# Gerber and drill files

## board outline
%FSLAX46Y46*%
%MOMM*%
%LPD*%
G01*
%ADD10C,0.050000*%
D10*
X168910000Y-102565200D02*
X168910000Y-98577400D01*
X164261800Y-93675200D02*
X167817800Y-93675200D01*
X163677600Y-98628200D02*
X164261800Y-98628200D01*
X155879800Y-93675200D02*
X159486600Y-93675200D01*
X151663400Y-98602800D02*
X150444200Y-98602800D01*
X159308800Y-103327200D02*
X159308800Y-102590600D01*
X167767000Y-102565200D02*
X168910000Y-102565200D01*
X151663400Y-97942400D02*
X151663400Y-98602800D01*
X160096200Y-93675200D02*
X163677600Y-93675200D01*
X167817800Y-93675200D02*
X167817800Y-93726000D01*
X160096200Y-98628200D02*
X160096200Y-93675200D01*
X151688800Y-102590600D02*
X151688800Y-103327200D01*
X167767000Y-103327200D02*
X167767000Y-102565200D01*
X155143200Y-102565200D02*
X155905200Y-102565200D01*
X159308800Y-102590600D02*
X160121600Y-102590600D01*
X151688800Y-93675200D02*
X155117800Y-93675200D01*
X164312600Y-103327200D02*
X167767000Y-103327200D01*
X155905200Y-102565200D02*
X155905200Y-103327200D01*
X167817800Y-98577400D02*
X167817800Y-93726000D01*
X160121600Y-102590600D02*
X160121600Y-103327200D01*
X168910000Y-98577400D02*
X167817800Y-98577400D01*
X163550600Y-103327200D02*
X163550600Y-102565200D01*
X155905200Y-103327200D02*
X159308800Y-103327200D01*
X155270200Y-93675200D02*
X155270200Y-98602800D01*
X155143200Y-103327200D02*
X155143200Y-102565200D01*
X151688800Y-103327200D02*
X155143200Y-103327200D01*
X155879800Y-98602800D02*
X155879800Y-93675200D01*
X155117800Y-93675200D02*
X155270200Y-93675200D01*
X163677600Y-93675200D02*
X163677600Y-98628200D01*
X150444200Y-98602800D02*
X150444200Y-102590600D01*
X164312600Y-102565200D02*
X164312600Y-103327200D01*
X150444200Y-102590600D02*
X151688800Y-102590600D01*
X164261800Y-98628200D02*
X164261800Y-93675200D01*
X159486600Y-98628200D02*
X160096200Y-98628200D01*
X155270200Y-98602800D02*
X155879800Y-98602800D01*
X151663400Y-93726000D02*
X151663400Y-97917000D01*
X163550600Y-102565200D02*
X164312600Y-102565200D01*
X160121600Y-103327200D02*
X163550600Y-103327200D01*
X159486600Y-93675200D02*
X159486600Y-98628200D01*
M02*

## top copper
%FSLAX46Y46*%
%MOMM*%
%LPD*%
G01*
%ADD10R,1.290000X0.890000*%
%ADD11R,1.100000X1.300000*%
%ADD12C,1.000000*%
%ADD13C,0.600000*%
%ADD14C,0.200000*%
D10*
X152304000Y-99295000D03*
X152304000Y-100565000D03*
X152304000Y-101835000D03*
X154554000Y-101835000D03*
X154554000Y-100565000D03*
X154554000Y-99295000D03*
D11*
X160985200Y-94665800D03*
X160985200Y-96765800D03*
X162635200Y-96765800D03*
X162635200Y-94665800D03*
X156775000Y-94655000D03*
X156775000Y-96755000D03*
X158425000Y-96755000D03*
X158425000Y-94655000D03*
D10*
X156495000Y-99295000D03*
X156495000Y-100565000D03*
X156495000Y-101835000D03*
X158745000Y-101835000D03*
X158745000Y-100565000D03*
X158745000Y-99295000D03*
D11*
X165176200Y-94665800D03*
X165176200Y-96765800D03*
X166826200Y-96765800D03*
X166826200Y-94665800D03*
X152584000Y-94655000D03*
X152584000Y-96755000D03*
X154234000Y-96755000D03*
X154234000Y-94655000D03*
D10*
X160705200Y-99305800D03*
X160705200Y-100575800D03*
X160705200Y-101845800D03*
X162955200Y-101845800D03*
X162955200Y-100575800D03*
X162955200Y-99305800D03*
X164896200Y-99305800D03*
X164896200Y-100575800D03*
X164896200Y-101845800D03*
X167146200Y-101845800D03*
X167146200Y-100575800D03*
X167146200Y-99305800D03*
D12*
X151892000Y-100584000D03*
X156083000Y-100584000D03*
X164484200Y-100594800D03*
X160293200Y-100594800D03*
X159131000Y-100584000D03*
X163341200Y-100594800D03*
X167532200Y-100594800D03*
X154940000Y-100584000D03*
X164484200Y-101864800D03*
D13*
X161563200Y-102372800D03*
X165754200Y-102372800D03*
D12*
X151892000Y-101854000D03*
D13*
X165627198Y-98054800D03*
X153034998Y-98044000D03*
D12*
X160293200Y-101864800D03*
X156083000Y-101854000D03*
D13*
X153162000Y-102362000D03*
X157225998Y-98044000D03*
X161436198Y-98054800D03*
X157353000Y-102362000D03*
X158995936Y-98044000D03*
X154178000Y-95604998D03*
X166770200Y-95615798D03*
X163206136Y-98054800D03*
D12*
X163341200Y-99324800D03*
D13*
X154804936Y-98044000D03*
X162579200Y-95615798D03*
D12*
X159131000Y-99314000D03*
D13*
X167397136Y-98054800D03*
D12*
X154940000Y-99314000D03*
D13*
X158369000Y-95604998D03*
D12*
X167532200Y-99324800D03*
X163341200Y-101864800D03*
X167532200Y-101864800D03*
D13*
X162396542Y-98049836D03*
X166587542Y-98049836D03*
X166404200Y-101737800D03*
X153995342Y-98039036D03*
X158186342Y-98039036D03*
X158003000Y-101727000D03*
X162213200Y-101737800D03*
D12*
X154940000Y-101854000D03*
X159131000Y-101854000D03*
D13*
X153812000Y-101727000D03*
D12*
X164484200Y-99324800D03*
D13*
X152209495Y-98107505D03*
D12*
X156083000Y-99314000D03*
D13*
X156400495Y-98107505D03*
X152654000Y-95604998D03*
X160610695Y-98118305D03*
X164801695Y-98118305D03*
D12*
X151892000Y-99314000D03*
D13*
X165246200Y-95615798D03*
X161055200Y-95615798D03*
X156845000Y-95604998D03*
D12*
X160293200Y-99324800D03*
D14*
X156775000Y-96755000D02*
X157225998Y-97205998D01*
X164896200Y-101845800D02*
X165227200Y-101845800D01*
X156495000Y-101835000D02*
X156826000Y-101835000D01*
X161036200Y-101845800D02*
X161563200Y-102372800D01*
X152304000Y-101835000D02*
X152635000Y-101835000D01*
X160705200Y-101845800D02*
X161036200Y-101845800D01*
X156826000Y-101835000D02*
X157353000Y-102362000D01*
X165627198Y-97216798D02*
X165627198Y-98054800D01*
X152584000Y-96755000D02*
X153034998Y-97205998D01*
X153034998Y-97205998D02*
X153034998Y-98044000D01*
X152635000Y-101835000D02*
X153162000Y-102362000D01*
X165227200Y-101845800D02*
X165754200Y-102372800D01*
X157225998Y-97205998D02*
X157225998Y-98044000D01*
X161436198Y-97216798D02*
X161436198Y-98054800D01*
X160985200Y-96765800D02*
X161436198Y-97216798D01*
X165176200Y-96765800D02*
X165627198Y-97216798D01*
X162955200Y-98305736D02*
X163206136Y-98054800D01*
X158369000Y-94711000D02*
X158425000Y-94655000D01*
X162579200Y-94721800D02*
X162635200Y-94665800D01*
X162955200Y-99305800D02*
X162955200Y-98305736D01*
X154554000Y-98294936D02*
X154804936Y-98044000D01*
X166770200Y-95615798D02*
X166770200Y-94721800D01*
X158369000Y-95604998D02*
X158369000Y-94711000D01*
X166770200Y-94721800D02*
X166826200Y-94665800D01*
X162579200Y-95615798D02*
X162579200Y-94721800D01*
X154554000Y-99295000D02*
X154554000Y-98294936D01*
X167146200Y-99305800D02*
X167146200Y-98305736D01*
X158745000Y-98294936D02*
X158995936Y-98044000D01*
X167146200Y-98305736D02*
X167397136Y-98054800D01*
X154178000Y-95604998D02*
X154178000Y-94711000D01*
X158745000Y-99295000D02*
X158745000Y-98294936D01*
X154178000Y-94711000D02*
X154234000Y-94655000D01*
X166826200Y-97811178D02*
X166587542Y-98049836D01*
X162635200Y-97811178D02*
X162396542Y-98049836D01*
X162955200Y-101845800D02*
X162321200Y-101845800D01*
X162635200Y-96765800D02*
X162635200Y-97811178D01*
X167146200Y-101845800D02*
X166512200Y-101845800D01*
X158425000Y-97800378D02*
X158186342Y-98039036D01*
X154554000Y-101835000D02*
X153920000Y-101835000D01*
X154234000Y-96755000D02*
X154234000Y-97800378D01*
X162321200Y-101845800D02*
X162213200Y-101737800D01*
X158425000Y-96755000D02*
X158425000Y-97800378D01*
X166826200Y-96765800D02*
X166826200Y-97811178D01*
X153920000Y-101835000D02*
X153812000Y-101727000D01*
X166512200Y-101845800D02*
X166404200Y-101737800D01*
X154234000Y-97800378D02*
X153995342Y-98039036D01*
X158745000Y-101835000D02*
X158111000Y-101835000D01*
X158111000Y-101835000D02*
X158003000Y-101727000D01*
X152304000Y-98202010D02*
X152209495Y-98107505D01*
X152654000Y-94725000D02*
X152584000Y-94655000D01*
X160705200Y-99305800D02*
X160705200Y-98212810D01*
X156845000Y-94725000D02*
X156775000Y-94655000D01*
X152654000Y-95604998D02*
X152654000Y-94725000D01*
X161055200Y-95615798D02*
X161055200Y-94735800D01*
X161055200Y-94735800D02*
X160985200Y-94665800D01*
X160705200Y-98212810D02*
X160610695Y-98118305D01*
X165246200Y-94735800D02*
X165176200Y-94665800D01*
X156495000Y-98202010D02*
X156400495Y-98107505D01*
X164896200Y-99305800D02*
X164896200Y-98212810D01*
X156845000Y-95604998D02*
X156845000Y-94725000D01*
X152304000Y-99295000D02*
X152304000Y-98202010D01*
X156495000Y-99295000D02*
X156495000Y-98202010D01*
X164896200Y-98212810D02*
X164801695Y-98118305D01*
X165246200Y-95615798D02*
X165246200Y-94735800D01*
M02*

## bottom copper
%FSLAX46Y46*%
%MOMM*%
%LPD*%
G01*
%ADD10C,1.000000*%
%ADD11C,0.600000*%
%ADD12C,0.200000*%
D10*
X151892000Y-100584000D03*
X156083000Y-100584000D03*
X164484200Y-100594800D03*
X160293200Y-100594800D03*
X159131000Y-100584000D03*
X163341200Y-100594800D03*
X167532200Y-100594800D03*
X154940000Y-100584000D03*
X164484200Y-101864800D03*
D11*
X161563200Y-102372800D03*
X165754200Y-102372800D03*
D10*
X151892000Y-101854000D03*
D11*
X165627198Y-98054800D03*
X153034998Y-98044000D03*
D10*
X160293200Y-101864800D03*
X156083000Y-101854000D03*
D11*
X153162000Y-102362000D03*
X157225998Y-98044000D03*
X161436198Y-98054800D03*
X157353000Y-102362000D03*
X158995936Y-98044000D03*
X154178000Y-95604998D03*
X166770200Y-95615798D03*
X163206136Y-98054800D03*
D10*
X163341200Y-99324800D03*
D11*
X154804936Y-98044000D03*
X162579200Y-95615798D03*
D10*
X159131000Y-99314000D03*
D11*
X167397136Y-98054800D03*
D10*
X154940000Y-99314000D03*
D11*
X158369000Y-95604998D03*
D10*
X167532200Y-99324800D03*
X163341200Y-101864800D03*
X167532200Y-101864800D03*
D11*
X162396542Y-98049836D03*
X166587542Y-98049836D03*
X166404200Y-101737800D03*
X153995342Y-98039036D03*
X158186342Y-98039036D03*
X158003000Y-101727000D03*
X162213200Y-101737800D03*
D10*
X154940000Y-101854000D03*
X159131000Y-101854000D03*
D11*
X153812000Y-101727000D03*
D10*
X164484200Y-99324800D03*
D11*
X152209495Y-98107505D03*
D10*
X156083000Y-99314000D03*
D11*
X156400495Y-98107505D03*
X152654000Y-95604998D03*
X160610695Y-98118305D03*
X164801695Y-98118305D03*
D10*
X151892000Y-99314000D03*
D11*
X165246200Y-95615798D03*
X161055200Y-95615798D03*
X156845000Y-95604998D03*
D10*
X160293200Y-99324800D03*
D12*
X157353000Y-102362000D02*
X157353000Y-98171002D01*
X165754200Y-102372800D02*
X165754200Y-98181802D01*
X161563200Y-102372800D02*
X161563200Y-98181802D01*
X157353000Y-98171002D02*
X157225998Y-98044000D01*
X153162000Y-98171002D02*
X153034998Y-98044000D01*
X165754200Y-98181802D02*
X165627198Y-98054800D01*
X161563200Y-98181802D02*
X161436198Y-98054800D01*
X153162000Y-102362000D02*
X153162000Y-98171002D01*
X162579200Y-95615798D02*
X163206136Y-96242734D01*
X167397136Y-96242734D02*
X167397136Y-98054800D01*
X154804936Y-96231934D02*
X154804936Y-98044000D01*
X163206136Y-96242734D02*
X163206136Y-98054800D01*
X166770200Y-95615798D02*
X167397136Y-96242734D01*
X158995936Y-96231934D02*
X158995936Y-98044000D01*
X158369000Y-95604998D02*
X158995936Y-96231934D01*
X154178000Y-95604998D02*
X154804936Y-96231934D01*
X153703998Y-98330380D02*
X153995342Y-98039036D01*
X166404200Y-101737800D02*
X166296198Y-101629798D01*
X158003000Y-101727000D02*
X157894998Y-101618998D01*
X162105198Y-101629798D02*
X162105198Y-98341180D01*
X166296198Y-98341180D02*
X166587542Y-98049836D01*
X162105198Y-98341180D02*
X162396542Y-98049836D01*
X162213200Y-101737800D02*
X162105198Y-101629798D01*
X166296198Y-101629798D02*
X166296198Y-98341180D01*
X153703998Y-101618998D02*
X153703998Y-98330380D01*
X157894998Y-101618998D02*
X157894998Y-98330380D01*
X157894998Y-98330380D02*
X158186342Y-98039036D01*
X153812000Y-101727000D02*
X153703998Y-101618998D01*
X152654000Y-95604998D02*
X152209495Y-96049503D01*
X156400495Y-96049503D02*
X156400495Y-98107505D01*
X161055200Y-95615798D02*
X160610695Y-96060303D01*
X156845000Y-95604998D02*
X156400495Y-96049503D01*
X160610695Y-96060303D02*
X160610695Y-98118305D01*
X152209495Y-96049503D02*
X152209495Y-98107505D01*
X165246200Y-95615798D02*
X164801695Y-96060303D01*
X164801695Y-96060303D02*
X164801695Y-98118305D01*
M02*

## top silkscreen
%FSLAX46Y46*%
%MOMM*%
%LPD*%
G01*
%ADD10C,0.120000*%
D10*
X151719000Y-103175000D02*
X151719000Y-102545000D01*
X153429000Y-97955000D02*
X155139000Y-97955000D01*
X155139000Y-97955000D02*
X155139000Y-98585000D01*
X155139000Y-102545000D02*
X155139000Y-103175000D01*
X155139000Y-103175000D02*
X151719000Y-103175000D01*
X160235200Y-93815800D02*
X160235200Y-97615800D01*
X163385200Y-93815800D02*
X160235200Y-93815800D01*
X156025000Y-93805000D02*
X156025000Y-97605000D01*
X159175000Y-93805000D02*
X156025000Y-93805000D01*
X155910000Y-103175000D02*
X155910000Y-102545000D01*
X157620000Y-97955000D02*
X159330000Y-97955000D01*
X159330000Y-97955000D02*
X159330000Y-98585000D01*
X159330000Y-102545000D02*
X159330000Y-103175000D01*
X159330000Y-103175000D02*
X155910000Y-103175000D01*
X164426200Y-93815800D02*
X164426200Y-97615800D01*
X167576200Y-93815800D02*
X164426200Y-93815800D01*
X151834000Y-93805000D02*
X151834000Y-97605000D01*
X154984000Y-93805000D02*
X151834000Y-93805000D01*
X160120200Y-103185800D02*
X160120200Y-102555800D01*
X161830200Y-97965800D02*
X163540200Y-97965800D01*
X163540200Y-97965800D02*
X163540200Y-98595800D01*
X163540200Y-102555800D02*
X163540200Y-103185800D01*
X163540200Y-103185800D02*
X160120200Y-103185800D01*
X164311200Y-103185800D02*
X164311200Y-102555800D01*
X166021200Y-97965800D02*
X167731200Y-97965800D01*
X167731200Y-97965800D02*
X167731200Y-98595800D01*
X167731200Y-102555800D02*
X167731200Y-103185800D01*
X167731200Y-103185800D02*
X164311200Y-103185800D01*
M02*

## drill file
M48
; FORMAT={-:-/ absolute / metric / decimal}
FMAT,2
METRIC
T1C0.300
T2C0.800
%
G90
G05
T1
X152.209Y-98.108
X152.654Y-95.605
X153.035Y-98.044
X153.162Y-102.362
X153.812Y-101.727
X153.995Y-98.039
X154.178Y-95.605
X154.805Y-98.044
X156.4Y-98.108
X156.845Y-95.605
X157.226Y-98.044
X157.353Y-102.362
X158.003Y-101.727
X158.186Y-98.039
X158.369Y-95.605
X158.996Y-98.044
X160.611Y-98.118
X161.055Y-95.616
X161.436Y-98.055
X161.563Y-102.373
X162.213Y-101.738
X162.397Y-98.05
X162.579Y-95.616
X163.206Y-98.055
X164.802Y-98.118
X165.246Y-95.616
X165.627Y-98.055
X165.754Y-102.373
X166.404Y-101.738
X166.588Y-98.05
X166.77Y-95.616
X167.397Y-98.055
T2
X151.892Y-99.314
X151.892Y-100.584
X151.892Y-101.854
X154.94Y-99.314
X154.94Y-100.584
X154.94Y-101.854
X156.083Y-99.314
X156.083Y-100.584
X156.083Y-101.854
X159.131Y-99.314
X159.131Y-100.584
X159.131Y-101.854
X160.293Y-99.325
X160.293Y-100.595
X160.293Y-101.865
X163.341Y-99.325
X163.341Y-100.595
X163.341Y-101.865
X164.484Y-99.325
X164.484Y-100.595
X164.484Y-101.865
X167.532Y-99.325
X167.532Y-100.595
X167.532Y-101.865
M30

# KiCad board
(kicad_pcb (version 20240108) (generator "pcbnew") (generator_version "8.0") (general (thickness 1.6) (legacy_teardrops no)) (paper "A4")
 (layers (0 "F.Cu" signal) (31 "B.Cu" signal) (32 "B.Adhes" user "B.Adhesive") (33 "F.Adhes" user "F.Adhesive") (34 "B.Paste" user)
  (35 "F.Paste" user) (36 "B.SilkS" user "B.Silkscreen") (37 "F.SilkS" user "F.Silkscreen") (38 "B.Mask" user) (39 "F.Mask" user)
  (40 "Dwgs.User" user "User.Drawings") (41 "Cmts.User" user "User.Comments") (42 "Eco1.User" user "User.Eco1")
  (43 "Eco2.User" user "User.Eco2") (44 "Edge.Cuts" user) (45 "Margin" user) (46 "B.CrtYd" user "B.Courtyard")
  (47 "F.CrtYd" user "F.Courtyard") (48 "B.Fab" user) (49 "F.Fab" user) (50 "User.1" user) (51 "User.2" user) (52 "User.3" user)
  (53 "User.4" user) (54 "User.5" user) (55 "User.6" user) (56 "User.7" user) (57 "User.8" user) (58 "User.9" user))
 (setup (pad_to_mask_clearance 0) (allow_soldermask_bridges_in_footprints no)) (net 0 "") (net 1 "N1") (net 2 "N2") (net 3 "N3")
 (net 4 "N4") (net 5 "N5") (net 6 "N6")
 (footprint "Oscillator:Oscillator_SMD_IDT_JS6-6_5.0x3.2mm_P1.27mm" (layer "F.Cu") (at 153.429 100.565)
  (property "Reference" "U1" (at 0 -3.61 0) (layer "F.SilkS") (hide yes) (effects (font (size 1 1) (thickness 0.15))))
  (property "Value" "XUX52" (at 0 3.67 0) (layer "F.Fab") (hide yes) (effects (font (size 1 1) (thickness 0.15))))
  (fp_line (start -1.71 2.61) (end -1.71 1.98) (stroke (width 0.12) (type solid)) (layer "F.SilkS"))
  (fp_line (start 0 -2.61) (end 1.71 -2.61) (stroke (width 0.12) (type solid)) (layer "F.SilkS"))
  (fp_line (start 1.71 -2.61) (end 1.71 -1.98) (stroke (width 0.12) (type solid)) (layer "F.SilkS"))
  (fp_line (start 1.71 1.98) (end 1.71 2.61) (stroke (width 0.12) (type solid)) (layer "F.SilkS"))
  (fp_line (start 1.71 2.61) (end -1.71 2.61) (stroke (width 0.12) (type solid)) (layer "F.SilkS"))
  (pad "1" smd rect (at -1.125 -1.27 270) (size 0.89 1.29) (layers "F.Cu" "F.Paste" "F.Mask") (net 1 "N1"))
  (pad "2" smd rect (at -1.125 0 270) (size 0.89 1.29) (layers "F.Cu" "F.Paste" "F.Mask") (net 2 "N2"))
  (pad "3" smd rect (at -1.125 1.27 270) (size 0.89 1.29) (layers "F.Cu" "F.Paste" "F.Mask") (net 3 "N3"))
  (pad "4" smd rect (at 1.125 1.27 270) (size 0.89 1.29) (layers "F.Cu" "F.Paste" "F.Mask") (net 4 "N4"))
  (pad "5" smd rect (at 1.125 0 270) (size 0.89 1.29) (layers "F.Cu" "F.Paste" "F.Mask") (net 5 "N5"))
  (pad "6" smd rect (at 1.125 -1.27 270) (size 0.89 1.29) (layers "F.Cu" "F.Paste" "F.Mask") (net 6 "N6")))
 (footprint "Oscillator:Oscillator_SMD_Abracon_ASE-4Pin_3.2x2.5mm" (layer "F.Cu") (at 161.8102 95.7158 -90)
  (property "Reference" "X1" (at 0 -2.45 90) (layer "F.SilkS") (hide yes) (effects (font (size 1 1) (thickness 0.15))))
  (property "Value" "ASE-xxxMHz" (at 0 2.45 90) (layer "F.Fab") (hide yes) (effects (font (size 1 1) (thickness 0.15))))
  (fp_line (start -1.9 1.575) (end 1.9 1.575) (stroke (width 0.12) (type solid)) (layer "F.SilkS"))
  (fp_line (start -1.9 -1.575) (end -1.9 1.575) (stroke (width 0.12) (type solid)) (layer "F.SilkS"))
  (pad "1" smd rect (at -1.05 0.825 270) (size 1.3 1.1) (layers "F.Cu" "F.Paste" "F.Mask") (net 1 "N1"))
  (pad "2" smd rect (at 1.05 0.825 270) (size 1.3 1.1) (layers "F.Cu" "F.Paste" "F.Mask") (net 3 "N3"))
  (pad "3" smd rect (at 1.05 -0.825 270) (size 1.3 1.1) (layers "F.Cu" "F.Paste" "F.Mask") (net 4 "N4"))
  (pad "4" smd rect (at -1.05 -0.825 270) (size 1.3 1.1) (layers "F.Cu" "F.Paste" "F.Mask") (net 6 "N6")))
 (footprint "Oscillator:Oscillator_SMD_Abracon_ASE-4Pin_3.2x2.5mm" (layer "F.Cu") (at 157.6 95.705 -90)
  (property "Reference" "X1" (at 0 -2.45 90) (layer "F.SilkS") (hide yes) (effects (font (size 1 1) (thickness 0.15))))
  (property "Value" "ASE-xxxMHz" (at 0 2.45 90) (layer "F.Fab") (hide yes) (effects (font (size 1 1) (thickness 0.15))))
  (fp_line (start -1.9 1.575) (end 1.9 1.575) (stroke (width 0.12) (type solid)) (layer "F.SilkS"))
  (fp_line (start -1.9 -1.575) (end -1.9 1.575) (stroke (width 0.12) (type solid)) (layer "F.SilkS"))
  (pad "1" smd rect (at -1.05 0.825 270) (size 1.3 1.1) (layers "F.Cu" "F.Paste" "F.Mask") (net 1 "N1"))
  (pad "2" smd rect (at 1.05 0.825 270) (size 1.3 1.1) (layers "F.Cu" "F.Paste" "F.Mask") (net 3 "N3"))
  (pad "3" smd rect (at 1.05 -0.825 270) (size 1.3 1.1) (layers "F.Cu" "F.Paste" "F.Mask") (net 4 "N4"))
  (pad "4" smd rect (at -1.05 -0.825 270) (size 1.3 1.1) (layers "F.Cu" "F.Paste" "F.Mask") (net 6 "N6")))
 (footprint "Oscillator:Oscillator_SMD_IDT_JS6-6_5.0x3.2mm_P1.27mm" (layer "F.Cu") (at 157.62 100.565)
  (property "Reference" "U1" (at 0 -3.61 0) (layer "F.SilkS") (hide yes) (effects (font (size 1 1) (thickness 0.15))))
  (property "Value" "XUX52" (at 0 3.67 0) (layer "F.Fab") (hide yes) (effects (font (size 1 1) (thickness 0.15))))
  (fp_line (start -1.71 2.61) (end -1.71 1.98) (stroke (width 0.12) (type solid)) (layer "F.SilkS"))
  (fp_line (start 0 -2.61) (end 1.71 -2.61) (stroke (width 0.12) (type solid)) (layer "F.SilkS"))
  (fp_line (start 1.71 -2.61) (end 1.71 -1.98) (stroke (width 0.12) (type solid)) (layer "F.SilkS"))
  (fp_line (start 1.71 1.98) (end 1.71 2.61) (stroke (width 0.12) (type solid)) (layer "F.SilkS"))
  (fp_line (start 1.71 2.61) (end -1.71 2.61) (stroke (width 0.12) (type solid)) (layer "F.SilkS"))
  (pad "1" smd rect (at -1.125 -1.27 270) (size 0.89 1.29) (layers "F.Cu" "F.Paste" "F.Mask") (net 1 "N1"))
  (pad "2" smd rect (at -1.125 0 270) (size 0.89 1.29) (layers "F.Cu" "F.Paste" "F.Mask") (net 2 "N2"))
  (pad "3" smd rect (at -1.125 1.27 270) (size 0.89 1.29) (layers "F.Cu" "F.Paste" "F.Mask") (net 3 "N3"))
  (pad "4" smd rect (at 1.125 1.27 270) (size 0.89 1.29) (layers "F.Cu" "F.Paste" "F.Mask") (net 4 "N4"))
  (pad "5" smd rect (at 1.125 0 270) (size 0.89 1.29) (layers "F.Cu" "F.Paste" "F.Mask") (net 5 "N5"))
  (pad "6" smd rect (at 1.125 -1.27 270) (size 0.89 1.29) (layers "F.Cu" "F.Paste" "F.Mask") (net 6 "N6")))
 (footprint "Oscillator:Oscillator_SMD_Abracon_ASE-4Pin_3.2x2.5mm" (layer "F.Cu") (at 166.0012 95.7158 -90)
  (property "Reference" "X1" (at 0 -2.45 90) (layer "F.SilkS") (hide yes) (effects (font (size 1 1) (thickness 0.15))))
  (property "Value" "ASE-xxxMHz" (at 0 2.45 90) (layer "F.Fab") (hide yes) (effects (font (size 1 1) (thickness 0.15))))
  (fp_line (start -1.9 1.575) (end 1.9 1.575) (stroke (width 0.12) (type solid)) (layer "F.SilkS"))
  (fp_line (start -1.9 -1.575) (end -1.9 1.575) (stroke (width 0.12) (type solid)) (layer "F.SilkS"))
  (pad "1" smd rect (at -1.05 0.825 270) (size 1.3 1.1) (layers "F.Cu" "F.Paste" "F.Mask") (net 1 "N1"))
  (pad "2" smd rect (at 1.05 0.825 270) (size 1.3 1.1) (layers "F.Cu" "F.Paste" "F.Mask") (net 3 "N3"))
  (pad "3" smd rect (at 1.05 -0.825 270) (size 1.3 1.1) (layers "F.Cu" "F.Paste" "F.Mask") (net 4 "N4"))
  (pad "4" smd rect (at -1.05 -0.825 270) (size 1.3 1.1) (layers "F.Cu" "F.Paste" "F.Mask") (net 6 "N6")))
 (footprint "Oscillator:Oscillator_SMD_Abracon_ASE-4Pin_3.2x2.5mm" (layer "F.Cu") (at 153.409 95.705 -90)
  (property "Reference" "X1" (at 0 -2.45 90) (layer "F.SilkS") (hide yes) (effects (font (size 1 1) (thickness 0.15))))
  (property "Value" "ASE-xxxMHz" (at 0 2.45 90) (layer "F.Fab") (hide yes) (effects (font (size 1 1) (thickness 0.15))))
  (fp_line (start -1.9 1.575) (end 1.9 1.575) (stroke (width 0.12) (type solid)) (layer "F.SilkS"))
  (fp_line (start -1.9 -1.575) (end -1.9 1.575) (stroke (width 0.12) (type solid)) (layer "F.SilkS"))
  (pad "1" smd rect (at -1.05 0.825 270) (size 1.3 1.1) (layers "F.Cu" "F.Paste" "F.Mask") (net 1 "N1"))
  (pad "2" smd rect (at 1.05 0.825 270) (size 1.3 1.1) (layers "F.Cu" "F.Paste" "F.Mask") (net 3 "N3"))
  (pad "3" smd rect (at 1.05 -0.825 270) (size 1.3 1.1) (layers "F.Cu" "F.Paste" "F.Mask") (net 4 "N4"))
  (pad "4" smd rect (at -1.05 -0.825 270) (size 1.3 1.1) (layers "F.Cu" "F.Paste" "F.Mask") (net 6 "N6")))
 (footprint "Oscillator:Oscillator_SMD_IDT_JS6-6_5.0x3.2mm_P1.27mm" (layer "F.Cu") (at 161.8302 100.5758)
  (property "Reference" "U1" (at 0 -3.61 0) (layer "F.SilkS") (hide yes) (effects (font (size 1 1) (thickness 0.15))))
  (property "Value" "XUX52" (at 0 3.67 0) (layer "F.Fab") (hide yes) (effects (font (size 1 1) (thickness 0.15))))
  (fp_line (start -1.71 2.61) (end -1.71 1.98) (stroke (width 0.12) (type solid)) (layer "F.SilkS"))
  (fp_line (start 0 -2.61) (end 1.71 -2.61) (stroke (width 0.12) (type solid)) (layer "F.SilkS"))
  (fp_line (start 1.71 -2.61) (end 1.71 -1.98) (stroke (width 0.12) (type solid)) (layer "F.SilkS"))
  (fp_line (start 1.71 1.98) (end 1.71 2.61) (stroke (width 0.12) (type solid)) (layer "F.SilkS"))
  (fp_line (start 1.71 2.61) (end -1.71 2.61) (stroke (width 0.12) (type solid)) (layer "F.SilkS"))
  (pad "1" smd rect (at -1.125 -1.27 270) (size 0.89 1.29) (layers "F.Cu" "F.Paste" "F.Mask") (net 1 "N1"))
  (pad "2" smd rect (at -1.125 0 270) (size 0.89 1.29) (layers "F.Cu" "F.Paste" "F.Mask") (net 2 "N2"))
  (pad "3" smd rect (at -1.125 1.27 270) (size 0.89 1.29) (layers "F.Cu" "F.Paste" "F.Mask") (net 3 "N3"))
  (pad "4" smd rect (at 1.125 1.27 270) (size 0.89 1.29) (layers "F.Cu" "F.Paste" "F.Mask") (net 4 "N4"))
  (pad "5" smd rect (at 1.125 0 270) (size 0.89 1.29) (layers "F.Cu" "F.Paste" "F.Mask") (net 5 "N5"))
  (pad "6" smd rect (at 1.125 -1.27 270) (size 0.89 1.29) (layers "F.Cu" "F.Paste" "F.Mask") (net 6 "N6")))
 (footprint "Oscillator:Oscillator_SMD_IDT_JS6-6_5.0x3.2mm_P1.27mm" (layer "F.Cu") (at 166.0212 100.5758)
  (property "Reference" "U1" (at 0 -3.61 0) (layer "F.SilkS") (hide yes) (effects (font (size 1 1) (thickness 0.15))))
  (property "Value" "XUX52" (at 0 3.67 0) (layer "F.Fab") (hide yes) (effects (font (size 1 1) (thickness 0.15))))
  (fp_line (start -1.71 2.61) (end -1.71 1.98) (stroke (width 0.12) (type solid)) (layer "F.SilkS"))
  (fp_line (start 0 -2.61) (end 1.71 -2.61) (stroke (width 0.12) (type solid)) (layer "F.SilkS"))
  (fp_line (start 1.71 -2.61) (end 1.71 -1.98) (stroke (width 0.12) (type solid)) (layer "F.SilkS"))
  (fp_line (start 1.71 1.98) (end 1.71 2.61) (stroke (width 0.12) (type solid)) (layer "F.SilkS"))
  (fp_line (start 1.71 2.61) (end -1.71 2.61) (stroke (width 0.12) (type solid)) (layer "F.SilkS"))
  (pad "1" smd rect (at -1.125 -1.27 270) (size 0.89 1.29) (layers "F.Cu" "F.Paste" "F.Mask") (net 1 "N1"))
  (pad "2" smd rect (at -1.125 0 270) (size 0.89 1.29) (layers "F.Cu" "F.Paste" "F.Mask") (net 2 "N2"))
  (pad "3" smd rect (at -1.125 1.27 270) (size 0.89 1.29) (layers "F.Cu" "F.Paste" "F.Mask") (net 3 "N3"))
  (pad "4" smd rect (at 1.125 1.27 270) (size 0.89 1.29) (layers "F.Cu" "F.Paste" "F.Mask") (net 4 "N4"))
  (pad "5" smd rect (at 1.125 0 270) (size 0.89 1.29) (layers "F.Cu" "F.Paste" "F.Mask") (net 5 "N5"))
  (pad "6" smd rect (at 1.125 -1.27 270) (size 0.89 1.29) (layers "F.Cu" "F.Paste" "F.Mask") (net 6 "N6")))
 (gr_line (start 168.91 102.5652) (end 168.91 98.5774) (stroke (width 0.05) (type default)) (layer "Edge.Cuts"))
 (gr_line (start 164.2618 93.6752) (end 167.8178 93.6752) (stroke (width 0.05) (type default)) (layer "Edge.Cuts"))
 (gr_line (start 163.6776 98.6282) (end 164.2618 98.6282) (stroke (width 0.05) (type default)) (layer "Edge.Cuts"))
 (gr_line (start 155.8798 93.6752) (end 159.4866 93.6752) (stroke (width 0.05) (type default)) (layer "Edge.Cuts"))
 (gr_line (start 151.6634 98.6028) (end 150.4442 98.6028) (stroke (width 0.05) (type default)) (layer "Edge.Cuts"))
 (gr_line (start 159.3088 103.3272) (end 159.3088 102.5906) (stroke (width 0.05) (type default)) (layer "Edge.Cuts"))
 (gr_line (start 167.767 102.5652) (end 168.91 102.5652) (stroke (width 0.05) (type default)) (layer "Edge.Cuts"))
 (gr_line (start 151.6634 97.9424) (end 151.6634 98.6028) (stroke (width 0.05) (type default)) (layer "Edge.Cuts"))
 (gr_line (start 160.0962 93.6752) (end 163.6776 93.6752) (stroke (width 0.05) (type default)) (layer "Edge.Cuts"))
 (gr_line (start 167.8178 93.6752) (end 167.8178 93.726) (stroke (width 0.05) (type default)) (layer "Edge.Cuts"))
 (gr_line (start 160.0962 98.6282) (end 160.0962 93.6752) (stroke (width 0.05) (type default)) (layer "Edge.Cuts"))
 (gr_line (start 151.6888 102.5906) (end 151.6888 103.3272) (stroke (width 0.05) (type default)) (layer "Edge.Cuts"))
 (gr_line (start 167.767 103.3272) (end 167.767 102.5652) (stroke (width 0.05) (type default)) (layer "Edge.Cuts"))
 (gr_line (start 155.1432 102.5652) (end 155.9052 102.5652) (stroke (width 0.05) (type default)) (layer "Edge.Cuts"))
 (gr_line (start 159.3088 102.5906) (end 160.1216 102.5906) (stroke (width 0.05) (type default)) (layer "Edge.Cuts"))
 (gr_line (start 151.6888 93.6752) (end 155.1178 93.6752) (stroke (width 0.05) (type default)) (layer "Edge.Cuts"))
 (gr_line (start 164.3126 103.3272) (end 167.767 103.3272) (stroke (width 0.05) (type default)) (layer "Edge.Cuts"))
 (gr_line (start 155.9052 102.5652) (end 155.9052 103.3272) (stroke (width 0.05) (type default)) (layer "Edge.Cuts"))
 (gr_line (start 167.8178 98.5774) (end 167.8178 93.726) (stroke (width 0.05) (type default)) (layer "Edge.Cuts"))
 (gr_line (start 160.1216 102.5906) (end 160.1216 103.3272) (stroke (width 0.05) (type default)) (layer "Edge.Cuts"))
 (gr_line (start 168.91 98.5774) (end 167.8178 98.5774) (stroke (width 0.05) (type default)) (layer "Edge.Cuts"))
 (gr_line (start 163.5506 103.3272) (end 163.5506 102.5652) (stroke (width 0.05) (type default)) (layer "Edge.Cuts"))
 (gr_line (start 155.9052 103.3272) (end 159.3088 103.3272) (stroke (width 0.05) (type default)) (layer "Edge.Cuts"))
 (gr_line (start 155.2702 93.6752) (end 155.2702 98.6028) (stroke (width 0.05) (type default)) (layer "Edge.Cuts"))
 (gr_line (start 155.1432 103.3272) (end 155.1432 102.5652) (stroke (width 0.05) (type default)) (layer "Edge.Cuts"))
 (gr_line (start 151.6888 103.3272) (end 155.1432 103.3272) (stroke (width 0.05) (type default)) (layer "Edge.Cuts"))
 (gr_line (start 155.8798 98.6028) (end 155.8798 93.6752) (stroke (width 0.05) (type default)) (layer "Edge.Cuts"))
 (gr_line (start 155.1178 93.6752) (end 155.2702 93.6752) (stroke (width 0.05) (type default)) (layer "Edge.Cuts"))
 (gr_line (start 163.6776 93.6752) (end 163.6776 98.6282) (stroke (width 0.05) (type default)) (layer "Edge.Cuts"))
 (gr_line (start 150.4442 98.6028) (end 150.4442 102.5906) (stroke (width 0.05) (type default)) (layer "Edge.Cuts"))
 (gr_line (start 164.3126 102.5652) (end 164.3126 103.3272) (stroke (width 0.05) (type default)) (layer "Edge.Cuts"))
 (gr_line (start 150.4442 102.5906) (end 151.6888 102.5906) (stroke (width 0.05) (type default)) (layer "Edge.Cuts"))
 (gr_line (start 164.2618 98.6282) (end 164.2618 93.6752) (stroke (width 0.05) (type default)) (layer "Edge.Cuts"))
 (gr_line (start 159.4866 98.6282) (end 160.0962 98.6282) (stroke (width 0.05) (type default)) (layer "Edge.Cuts"))
 (gr_line (start 155.2702 98.6028) (end 155.8798 98.6028) (stroke (width 0.05) (type default)) (layer "Edge.Cuts"))
 (gr_line (start 151.6634 93.726) (end 151.6634 97.917) (stroke (width 0.05) (type default)) (layer "Edge.Cuts"))
 (gr_line (start 163.5506 102.5652) (end 164.3126 102.5652) (stroke (width 0.05) (type default)) (layer "Edge.Cuts"))
 (gr_line (start 160.1216 103.3272) (end 163.5506 103.3272) (stroke (width 0.05) (type default)) (layer "Edge.Cuts"))
 (gr_line (start 159.4866 93.6752) (end 159.4866 98.6282) (stroke (width 0.05) (type default)) (layer "Edge.Cuts"))
 (via (at 151.892 100.584) (size 1) (drill 0.8) (layers "F.Cu" "B.Cu") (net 2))
 (via (at 156.083 100.584) (size 1) (drill 0.8) (layers "F.Cu" "B.Cu") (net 2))
 (via (at 164.4842 100.5948) (size 1) (drill 0.8) (layers "F.Cu" "B.Cu") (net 2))
 (via (at 160.2932 100.5948) (size 1) (drill 0.8) (layers "F.Cu" "B.Cu") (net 2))
 (via (at 159.131 100.584) (size 1) (drill 0.8) (layers "F.Cu" "B.Cu") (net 5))
 (via (at 163.3412 100.5948) (size 1) (drill 0.8) (layers "F.Cu" "B.Cu") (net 5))
 (via (at 167.5322 100.5948) (size 1) (drill 0.8) (layers "F.Cu" "B.Cu") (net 5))
 (via (at 154.94 100.584) (size 1) (drill 0.8) (layers "F.Cu" "B.Cu") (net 5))
 (segment (start 156.775 96.755) (end 157.225998 97.205998) (width 0.2) (layer "F.Cu") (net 3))
 (segment (start 164.8962 101.8458) (end 165.2272 101.8458) (width 0.2) (layer "F.Cu") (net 3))
 (segment (start 156.495 101.835) (end 156.826 101.835) (width 0.2) (layer "F.Cu") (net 3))
 (segment (start 161.0362 101.8458) (end 161.5632 102.3728) (width 0.2) (layer "F.Cu") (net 3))
 (segment (start 152.304 101.835) (end 152.635 101.835) (width 0.2) (layer "F.Cu") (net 3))
 (segment (start 160.7052 101.8458) (end 161.0362 101.8458) (width 0.2) (layer "F.Cu") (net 3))
 (segment (start 156.826 101.835) (end 157.353 102.362) (width 0.2) (layer "F.Cu") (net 3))
 (segment (start 165.627198 97.216798) (end 165.627198 98.0548) (width 0.2) (layer "F.Cu") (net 3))
 (segment (start 152.584 96.755) (end 153.034998 97.205998) (width 0.2) (layer "F.Cu") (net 3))
 (segment (start 153.034998 97.205998) (end 153.034998 98.044) (width 0.2) (layer "F.Cu") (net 3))
 (segment (start 152.635 101.835) (end 153.162 102.362) (width 0.2) (layer "F.Cu") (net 3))
 (segment (start 165.2272 101.8458) (end 165.7542 102.3728) (width 0.2) (layer "F.Cu") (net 3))
 (segment (start 157.225998 97.205998) (end 157.225998 98.044) (width 0.2) (layer "F.Cu") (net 3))
 (segment (start 161.436198 97.216798) (end 161.436198 98.0548) (width 0.2) (layer "F.Cu") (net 3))
 (segment (start 160.9852 96.7658) (end 161.436198 97.216798) (width 0.2) (layer "F.Cu") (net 3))
 (segment (start 165.1762 96.7658) (end 165.627198 97.216798) (width 0.2) (layer "F.Cu") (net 3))
 (via (at 164.4842 101.8648) (size 1) (drill 0.8) (layers "F.Cu" "B.Cu") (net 3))
 (via (at 161.5632 102.3728) (size 0.6) (drill 0.3) (layers "F.Cu" "B.Cu") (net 3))
 (via (at 165.7542 102.3728) (size 0.6) (drill 0.3) (layers "F.Cu" "B.Cu") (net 3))
 (via (at 151.892 101.854) (size 1) (drill 0.8) (layers "F.Cu" "B.Cu") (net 3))
 (via (at 165.627198 98.0548) (size 0.6) (drill 0.3) (layers "F.Cu" "B.Cu") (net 3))
 (via (at 153.034998 98.044) (size 0.6) (drill 0.3) (layers "F.Cu" "B.Cu") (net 3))
 (via (at 160.2932 101.8648) (size 1) (drill 0.8) (layers "F.Cu" "B.Cu") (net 3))
 (via (at 156.083 101.854) (size 1) (drill 0.8) (layers "F.Cu" "B.Cu") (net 3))
 (via (at 153.162 102.362) (size 0.6) (drill 0.3) (layers "F.Cu" "B.Cu") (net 3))
 (via (at 157.225998 98.044) (size 0.6) (drill 0.3) (layers "F.Cu" "B.Cu") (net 3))
 (via (at 161.436198 98.0548) (size 0.6) (drill 0.3) (layers "F.Cu" "B.Cu") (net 3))
 (via (at 157.353 102.362) (size 0.6) (drill 0.3) (layers "F.Cu" "B.Cu") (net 3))
 (segment (start 157.353 102.362) (end 157.353 98.171002) (width 0.2) (layer "B.Cu") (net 3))
 (segment (start 165.7542 102.3728) (end 165.7542 98.181802) (width 0.2) (layer "B.Cu") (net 3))
 (segment (start 161.5632 102.3728) (end 161.5632 98.181802) (width 0.2) (layer "B.Cu") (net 3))
 (segment (start 157.353 98.171002) (end 157.225998 98.044) (width 0.2) (layer "B.Cu") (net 3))
 (segment (start 153.162 98.171002) (end 153.034998 98.044) (width 0.2) (layer "B.Cu") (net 3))
 (segment (start 165.7542 98.181802) (end 165.627198 98.0548) (width 0.2) (layer "B.Cu") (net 3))
 (segment (start 161.5632 98.181802) (end 161.436198 98.0548) (width 0.2) (layer "B.Cu") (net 3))
 (segment (start 153.162 102.362) (end 153.162 98.171002) (width 0.2) (layer "B.Cu") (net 3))
 (segment (start 162.9552 98.305736) (end 163.206136 98.0548) (width 0.2) (layer "F.Cu") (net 6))
 (segment (start 158.369 94.711) (end 158.425 94.655) (width 0.2) (layer "F.Cu") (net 6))
 (segment (start 162.5792 94.7218) (end 162.6352 94.6658) (width 0.2) (layer "F.Cu") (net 6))
 (segment (start 162.9552 99.3058) (end 162.9552 98.305736) (width 0.2) (layer "F.Cu") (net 6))
 (segment (start 154.554 98.294936) (end 154.804936 98.044) (width 0.2) (layer "F.Cu") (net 6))
 (segment (start 166.7702 95.615798) (end 166.7702 94.7218) (width 0.2) (layer "F.Cu") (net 6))
 (segment (start 158.369 95.604998) (end 158.369 94.711) (width 0.2) (layer "F.Cu") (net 6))
 (segment (start 166.7702 94.7218) (end 166.8262 94.6658) (width 0.2) (layer "F.Cu") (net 6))
 (segment (start 162.5792 95.615798) (end 162.5792 94.7218) (width 0.2) (layer "F.Cu") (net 6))
 (segment (start 154.554 99.295) (end 154.554 98.294936) (width 0.2) (layer "F.Cu") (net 6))
 (segment (start 167.1462 99.3058) (end 167.1462 98.305736) (width 0.2) (layer "F.Cu") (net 6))
 (segment (start 158.745 98.294936) (end 158.995936 98.044) (width 0.2) (layer "F.Cu") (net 6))
 (segment (start 167.1462 98.305736) (end 167.397136 98.0548) (width 0.2) (layer "F.Cu") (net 6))
 (segment (start 154.178 95.604998) (end 154.178 94.711) (width 0.2) (layer "F.Cu") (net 6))
 (segment (start 158.745 99.295) (end 158.745 98.294936) (width 0.2) (layer "F.Cu") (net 6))
 (segment (start 154.178 94.711) (end 154.234 94.655) (width 0.2) (layer "F.Cu") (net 6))
 (via (at 158.995936 98.044) (size 0.6) (drill 0.3) (layers "F.Cu" "B.Cu") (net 6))
 (via (at 154.178 95.604998) (size 0.6) (drill 0.3) (layers "F.Cu" "B.Cu") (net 6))
 (via (at 166.7702 95.615798) (size 0.6) (drill 0.3) (layers "F.Cu" "B.Cu") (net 6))
 (via (at 163.206136 98.0548) (size 0.6) (drill 0.3) (layers "F.Cu" "B.Cu") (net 6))
 (via (at 163.3412 99.3248) (size 1) (drill 0.8) (layers "F.Cu" "B.Cu") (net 6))
 (via (at 154.804936 98.044) (size 0.6) (drill 0.3) (layers "F.Cu" "B.Cu") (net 6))
 (via (at 162.5792 95.615798) (size 0.6) (drill 0.3) (layers "F.Cu" "B.Cu") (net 6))
 (via (at 159.131 99.314) (size 1) (drill 0.8) (layers "F.Cu" "B.Cu") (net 6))
 (via (at 167.397136 98.0548) (size 0.6) (drill 0.3) (layers "F.Cu" "B.Cu") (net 6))
 (via (at 154.94 99.314) (size 1) (drill 0.8) (layers "F.Cu" "B.Cu") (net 6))
 (via (at 158.369 95.604998) (size 0.6) (drill 0.3) (layers "F.Cu" "B.Cu") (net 6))
 (via (at 167.5322 99.3248) (size 1) (drill 0.8) (layers "F.Cu" "B.Cu") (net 6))
 (segment (start 162.5792 95.615798) (end 163.206136 96.242734) (width 0.2) (layer "B.Cu") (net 6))
 (segment (start 167.397136 96.242734) (end 167.397136 98.0548) (width 0.2) (layer "B.Cu") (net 6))
 (segment (start 154.804936 96.231934) (end 154.804936 98.044) (width 0.2) (layer "B.Cu") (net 6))
 (segment (start 163.206136 96.242734) (end 163.206136 98.0548) (width 0.2) (layer "B.Cu") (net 6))
 (segment (start 166.7702 95.615798) (end 167.397136 96.242734) (width 0.2) (layer "B.Cu") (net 6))
 (segment (start 158.995936 96.231934) (end 158.995936 98.044) (width 0.2) (layer "B.Cu") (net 6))
 (segment (start 158.369 95.604998) (end 158.995936 96.231934) (width 0.2) (layer "B.Cu") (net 6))
 (segment (start 154.178 95.604998) (end 154.804936 96.231934) (width 0.2) (layer "B.Cu") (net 6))
 (segment (start 166.8262 97.811178) (end 166.587542 98.049836) (width 0.2) (layer "F.Cu") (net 4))
 (segment (start 162.6352 97.811178) (end 162.396542 98.049836) (width 0.2) (layer "F.Cu") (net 4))
 (segment (start 162.9552 101.8458) (end 162.3212 101.8458) (width 0.2) (layer "F.Cu") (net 4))
 (segment (start 162.6352 96.7658) (end 162.6352 97.811178) (width 0.2) (layer "F.Cu") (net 4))
 (segment (start 167.1462 101.8458) (end 166.5122 101.8458) (width 0.2) (layer "F.Cu") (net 4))
 (segment (start 158.425 97.800378) (end 158.186342 98.039036) (width 0.2) (layer "F.Cu") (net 4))
 (segment (start 154.554 101.835) (end 153.92 101.835) (width 0.2) (layer "F.Cu") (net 4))
 (segment (start 154.234 96.755) (end 154.234 97.800378) (width 0.2) (layer "F.Cu") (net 4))
 (segment (start 162.3212 101.8458) (end 162.2132 101.7378) (width 0.2) (layer "F.Cu") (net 4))
 (segment (start 158.425 96.755) (end 158.425 97.800378) (width 0.2) (layer "F.Cu") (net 4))
 (segment (start 166.8262 96.7658) (end 166.8262 97.811178) (width 0.2) (layer "F.Cu") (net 4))
 (segment (start 153.92 101.835) (end 153.812 101.727) (width 0.2) (layer "F.Cu") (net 4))
 (segment (start 166.5122 101.8458) (end 166.4042 101.7378) (width 0.2) (layer "F.Cu") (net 4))
 (segment (start 154.234 97.800378) (end 153.995342 98.039036) (width 0.2) (layer "F.Cu") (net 4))
 (segment (start 158.745 101.835) (end 158.111 101.835) (width 0.2) (layer "F.Cu") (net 4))
 (segment (start 158.111 101.835) (end 158.003 101.727) (width 0.2) (layer "F.Cu") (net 4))
 (via (at 163.3412 101.8648) (size 1) (drill 0.8) (layers "F.Cu" "B.Cu") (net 4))
 (via (at 167.5322 101.8648) (size 1) (drill 0.8) (layers "F.Cu" "B.Cu") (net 4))
 (via (at 162.396542 98.049836) (size 0.6) (drill 0.3) (layers "F.Cu" "B.Cu") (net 4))
 (via (at 166.587542 98.049836) (size 0.6) (drill 0.3) (layers "F.Cu" "B.Cu") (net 4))
 (via (at 166.4042 101.7378) (size 0.6) (drill 0.3) (layers "F.Cu" "B.Cu") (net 4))
 (via (at 153.995342 98.039036) (size 0.6) (drill 0.3) (layers "F.Cu" "B.Cu") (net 4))
 (via (at 158.186342 98.039036) (size 0.6) (drill 0.3) (layers "F.Cu" "B.Cu") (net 4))
 (via (at 158.003 101.727) (size 0.6) (drill 0.3) (layers "F.Cu" "B.Cu") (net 4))
 (via (at 162.2132 101.7378) (size 0.6) (drill 0.3) (layers "F.Cu" "B.Cu") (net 4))
 (via (at 154.94 101.854) (size 1) (drill 0.8) (layers "F.Cu" "B.Cu") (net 4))
 (via (at 159.131 101.854) (size 1) (drill 0.8) (layers "F.Cu" "B.Cu") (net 4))
 (via (at 153.812 101.727) (size 0.6) (drill 0.3) (layers "F.Cu" "B.Cu") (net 4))
 (segment (start 153.703998 98.33038) (end 153.995342 98.039036) (width 0.2) (layer "B.Cu") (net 4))
 (segment (start 166.4042 101.7378) (end 166.296198 101.629798) (width 0.2) (layer "B.Cu") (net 4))
 (segment (start 158.003 101.727) (end 157.894998 101.618998) (width 0.2) (layer "B.Cu") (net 4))
 (segment (start 162.105198 101.629798) (end 162.105198 98.34118) (width 0.2) (layer "B.Cu") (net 4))
 (segment (start 166.296198 98.34118) (end 166.587542 98.049836) (width 0.2) (layer "B.Cu") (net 4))
 (segment (start 162.105198 98.34118) (end 162.396542 98.049836) (width 0.2) (layer "B.Cu") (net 4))
 (segment (start 162.2132 101.7378) (end 162.105198 101.629798) (width 0.2) (layer "B.Cu") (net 4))
 (segment (start 166.296198 101.629798) (end 166.296198 98.34118) (width 0.2) (layer "B.Cu") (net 4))
 (segment (start 153.703998 101.618998) (end 153.703998 98.33038) (width 0.2) (layer "B.Cu") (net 4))
 (segment (start 157.894998 101.618998) (end 157.894998 98.33038) (width 0.2) (layer "B.Cu") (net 4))
 (segment (start 157.894998 98.33038) (end 158.186342 98.039036) (width 0.2) (layer "B.Cu") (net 4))
 (segment (start 153.812 101.727) (end 153.703998 101.618998) (width 0.2) (layer "B.Cu") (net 4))
 (segment (start 152.304 98.20201) (end 152.209495 98.107505) (width 0.2) (layer "F.Cu") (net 1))
 (segment (start 152.654 94.725) (end 152.584 94.655) (width 0.2) (layer "F.Cu") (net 1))
 (segment (start 160.7052 99.3058) (end 160.7052 98.21281) (width 0.2) (layer "F.Cu") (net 1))
 (segment (start 156.845 94.725) (end 156.775 94.655) (width 0.2) (layer "F.Cu") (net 1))
 (segment (start 152.654 95.604998) (end 152.654 94.725) (width 0.2) (layer "F.Cu") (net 1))
 (segment (start 161.0552 95.615798) (end 161.0552 94.7358) (width 0.2) (layer "F.Cu") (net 1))
 (segment (start 161.0552 94.7358) (end 160.9852 94.6658) (width 0.2) (layer "F.Cu") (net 1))
 (segment (start 160.7052 98.21281) (end 160.610695 98.118305) (width 0.2) (layer "F.Cu") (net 1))
 (segment (start 165.2462 94.7358) (end 165.1762 94.6658) (width 0.2) (layer "F.Cu") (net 1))
 (segment (start 156.495 98.20201) (end 156.400495 98.107505) (width 0.2) (layer "F.Cu") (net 1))
 (segment (start 164.8962 99.3058) (end 164.8962 98.21281) (width 0.2) (layer "F.Cu") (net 1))
 (segment (start 156.845 95.604998) (end 156.845 94.725) (width 0.2) (layer "F.Cu") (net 1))
 (segment (start 152.304 99.295) (end 152.304 98.20201) (width 0.2) (layer "F.Cu") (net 1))
 (segment (start 156.495 99.295) (end 156.495 98.20201) (width 0.2) (layer "F.Cu") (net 1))
 (segment (start 164.8962 98.21281) (end 164.801695 98.118305) (width 0.2) (layer "F.Cu") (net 1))
 (segment (start 165.2462 95.615798) (end 165.2462 94.7358) (width 0.2) (layer "F.Cu") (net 1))
 (via (at 164.4842 99.3248) (size 1) (drill 0.8) (layers "F.Cu" "B.Cu") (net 1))
 (via (at 152.209495 98.107505) (size 0.6) (drill 0.3) (layers "F.Cu" "B.Cu") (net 1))
 (via (at 156.083 99.314) (size 1) (drill 0.8) (layers "F.Cu" "B.Cu") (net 1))
 (via (at 156.400495 98.107505) (size 0.6) (drill 0.3) (layers "F.Cu" "B.Cu") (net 1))
 (via (at 152.654 95.604998) (size 0.6) (drill 0.3) (layers "F.Cu" "B.Cu") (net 1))
 (via (at 160.610695 98.118305) (size 0.6) (drill 0.3) (layers "F.Cu" "B.Cu") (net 1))
 (via (at 164.801695 98.118305) (size 0.6) (drill 0.3) (layers "F.Cu" "B.Cu") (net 1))
 (via (at 151.892 99.314) (size 1) (drill 0.8) (layers "F.Cu" "B.Cu") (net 1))
 (via (at 165.2462 95.615798) (size 0.6) (drill 0.3) (layers "F.Cu" "B.Cu") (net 1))
 (via (at 161.0552 95.615798) (size 0.6) (drill 0.3) (layers "F.Cu" "B.Cu") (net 1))
 (via (at 156.845 95.604998) (size 0.6) (drill 0.3) (layers "F.Cu" "B.Cu") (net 1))
 (via (at 160.2932 99.3248) (size 1) (drill 0.8) (layers "F.Cu" "B.Cu") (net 1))
 (segment (start 152.654 95.604998) (end 152.209495 96.049503) (width 0.2) (layer "B.Cu") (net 1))
 (segment (start 156.400495 96.049503) (end 156.400495 98.107505) (width 0.2) (layer "B.Cu") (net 1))
 (segment (start 161.0552 95.615798) (end 160.610695 96.060303) (width 0.2) (layer "B.Cu") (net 1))
 (segment (start 156.845 95.604998) (end 156.400495 96.049503) (width 0.2) (layer "B.Cu") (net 1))
 (segment (start 160.610695 96.060303) (end 160.610695 98.118305) (width 0.2) (layer "B.Cu") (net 1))
 (segment (start 152.209495 96.049503) (end 152.209495 98.107505) (width 0.2) (layer "B.Cu") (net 1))
 (segment (start 165.2462 95.615798) (end 164.801695 96.060303) (width 0.2) (layer "B.Cu") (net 1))
 (segment (start 164.801695 96.060303) (end 164.801695 98.118305) (width 0.2) (layer "B.Cu") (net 1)))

